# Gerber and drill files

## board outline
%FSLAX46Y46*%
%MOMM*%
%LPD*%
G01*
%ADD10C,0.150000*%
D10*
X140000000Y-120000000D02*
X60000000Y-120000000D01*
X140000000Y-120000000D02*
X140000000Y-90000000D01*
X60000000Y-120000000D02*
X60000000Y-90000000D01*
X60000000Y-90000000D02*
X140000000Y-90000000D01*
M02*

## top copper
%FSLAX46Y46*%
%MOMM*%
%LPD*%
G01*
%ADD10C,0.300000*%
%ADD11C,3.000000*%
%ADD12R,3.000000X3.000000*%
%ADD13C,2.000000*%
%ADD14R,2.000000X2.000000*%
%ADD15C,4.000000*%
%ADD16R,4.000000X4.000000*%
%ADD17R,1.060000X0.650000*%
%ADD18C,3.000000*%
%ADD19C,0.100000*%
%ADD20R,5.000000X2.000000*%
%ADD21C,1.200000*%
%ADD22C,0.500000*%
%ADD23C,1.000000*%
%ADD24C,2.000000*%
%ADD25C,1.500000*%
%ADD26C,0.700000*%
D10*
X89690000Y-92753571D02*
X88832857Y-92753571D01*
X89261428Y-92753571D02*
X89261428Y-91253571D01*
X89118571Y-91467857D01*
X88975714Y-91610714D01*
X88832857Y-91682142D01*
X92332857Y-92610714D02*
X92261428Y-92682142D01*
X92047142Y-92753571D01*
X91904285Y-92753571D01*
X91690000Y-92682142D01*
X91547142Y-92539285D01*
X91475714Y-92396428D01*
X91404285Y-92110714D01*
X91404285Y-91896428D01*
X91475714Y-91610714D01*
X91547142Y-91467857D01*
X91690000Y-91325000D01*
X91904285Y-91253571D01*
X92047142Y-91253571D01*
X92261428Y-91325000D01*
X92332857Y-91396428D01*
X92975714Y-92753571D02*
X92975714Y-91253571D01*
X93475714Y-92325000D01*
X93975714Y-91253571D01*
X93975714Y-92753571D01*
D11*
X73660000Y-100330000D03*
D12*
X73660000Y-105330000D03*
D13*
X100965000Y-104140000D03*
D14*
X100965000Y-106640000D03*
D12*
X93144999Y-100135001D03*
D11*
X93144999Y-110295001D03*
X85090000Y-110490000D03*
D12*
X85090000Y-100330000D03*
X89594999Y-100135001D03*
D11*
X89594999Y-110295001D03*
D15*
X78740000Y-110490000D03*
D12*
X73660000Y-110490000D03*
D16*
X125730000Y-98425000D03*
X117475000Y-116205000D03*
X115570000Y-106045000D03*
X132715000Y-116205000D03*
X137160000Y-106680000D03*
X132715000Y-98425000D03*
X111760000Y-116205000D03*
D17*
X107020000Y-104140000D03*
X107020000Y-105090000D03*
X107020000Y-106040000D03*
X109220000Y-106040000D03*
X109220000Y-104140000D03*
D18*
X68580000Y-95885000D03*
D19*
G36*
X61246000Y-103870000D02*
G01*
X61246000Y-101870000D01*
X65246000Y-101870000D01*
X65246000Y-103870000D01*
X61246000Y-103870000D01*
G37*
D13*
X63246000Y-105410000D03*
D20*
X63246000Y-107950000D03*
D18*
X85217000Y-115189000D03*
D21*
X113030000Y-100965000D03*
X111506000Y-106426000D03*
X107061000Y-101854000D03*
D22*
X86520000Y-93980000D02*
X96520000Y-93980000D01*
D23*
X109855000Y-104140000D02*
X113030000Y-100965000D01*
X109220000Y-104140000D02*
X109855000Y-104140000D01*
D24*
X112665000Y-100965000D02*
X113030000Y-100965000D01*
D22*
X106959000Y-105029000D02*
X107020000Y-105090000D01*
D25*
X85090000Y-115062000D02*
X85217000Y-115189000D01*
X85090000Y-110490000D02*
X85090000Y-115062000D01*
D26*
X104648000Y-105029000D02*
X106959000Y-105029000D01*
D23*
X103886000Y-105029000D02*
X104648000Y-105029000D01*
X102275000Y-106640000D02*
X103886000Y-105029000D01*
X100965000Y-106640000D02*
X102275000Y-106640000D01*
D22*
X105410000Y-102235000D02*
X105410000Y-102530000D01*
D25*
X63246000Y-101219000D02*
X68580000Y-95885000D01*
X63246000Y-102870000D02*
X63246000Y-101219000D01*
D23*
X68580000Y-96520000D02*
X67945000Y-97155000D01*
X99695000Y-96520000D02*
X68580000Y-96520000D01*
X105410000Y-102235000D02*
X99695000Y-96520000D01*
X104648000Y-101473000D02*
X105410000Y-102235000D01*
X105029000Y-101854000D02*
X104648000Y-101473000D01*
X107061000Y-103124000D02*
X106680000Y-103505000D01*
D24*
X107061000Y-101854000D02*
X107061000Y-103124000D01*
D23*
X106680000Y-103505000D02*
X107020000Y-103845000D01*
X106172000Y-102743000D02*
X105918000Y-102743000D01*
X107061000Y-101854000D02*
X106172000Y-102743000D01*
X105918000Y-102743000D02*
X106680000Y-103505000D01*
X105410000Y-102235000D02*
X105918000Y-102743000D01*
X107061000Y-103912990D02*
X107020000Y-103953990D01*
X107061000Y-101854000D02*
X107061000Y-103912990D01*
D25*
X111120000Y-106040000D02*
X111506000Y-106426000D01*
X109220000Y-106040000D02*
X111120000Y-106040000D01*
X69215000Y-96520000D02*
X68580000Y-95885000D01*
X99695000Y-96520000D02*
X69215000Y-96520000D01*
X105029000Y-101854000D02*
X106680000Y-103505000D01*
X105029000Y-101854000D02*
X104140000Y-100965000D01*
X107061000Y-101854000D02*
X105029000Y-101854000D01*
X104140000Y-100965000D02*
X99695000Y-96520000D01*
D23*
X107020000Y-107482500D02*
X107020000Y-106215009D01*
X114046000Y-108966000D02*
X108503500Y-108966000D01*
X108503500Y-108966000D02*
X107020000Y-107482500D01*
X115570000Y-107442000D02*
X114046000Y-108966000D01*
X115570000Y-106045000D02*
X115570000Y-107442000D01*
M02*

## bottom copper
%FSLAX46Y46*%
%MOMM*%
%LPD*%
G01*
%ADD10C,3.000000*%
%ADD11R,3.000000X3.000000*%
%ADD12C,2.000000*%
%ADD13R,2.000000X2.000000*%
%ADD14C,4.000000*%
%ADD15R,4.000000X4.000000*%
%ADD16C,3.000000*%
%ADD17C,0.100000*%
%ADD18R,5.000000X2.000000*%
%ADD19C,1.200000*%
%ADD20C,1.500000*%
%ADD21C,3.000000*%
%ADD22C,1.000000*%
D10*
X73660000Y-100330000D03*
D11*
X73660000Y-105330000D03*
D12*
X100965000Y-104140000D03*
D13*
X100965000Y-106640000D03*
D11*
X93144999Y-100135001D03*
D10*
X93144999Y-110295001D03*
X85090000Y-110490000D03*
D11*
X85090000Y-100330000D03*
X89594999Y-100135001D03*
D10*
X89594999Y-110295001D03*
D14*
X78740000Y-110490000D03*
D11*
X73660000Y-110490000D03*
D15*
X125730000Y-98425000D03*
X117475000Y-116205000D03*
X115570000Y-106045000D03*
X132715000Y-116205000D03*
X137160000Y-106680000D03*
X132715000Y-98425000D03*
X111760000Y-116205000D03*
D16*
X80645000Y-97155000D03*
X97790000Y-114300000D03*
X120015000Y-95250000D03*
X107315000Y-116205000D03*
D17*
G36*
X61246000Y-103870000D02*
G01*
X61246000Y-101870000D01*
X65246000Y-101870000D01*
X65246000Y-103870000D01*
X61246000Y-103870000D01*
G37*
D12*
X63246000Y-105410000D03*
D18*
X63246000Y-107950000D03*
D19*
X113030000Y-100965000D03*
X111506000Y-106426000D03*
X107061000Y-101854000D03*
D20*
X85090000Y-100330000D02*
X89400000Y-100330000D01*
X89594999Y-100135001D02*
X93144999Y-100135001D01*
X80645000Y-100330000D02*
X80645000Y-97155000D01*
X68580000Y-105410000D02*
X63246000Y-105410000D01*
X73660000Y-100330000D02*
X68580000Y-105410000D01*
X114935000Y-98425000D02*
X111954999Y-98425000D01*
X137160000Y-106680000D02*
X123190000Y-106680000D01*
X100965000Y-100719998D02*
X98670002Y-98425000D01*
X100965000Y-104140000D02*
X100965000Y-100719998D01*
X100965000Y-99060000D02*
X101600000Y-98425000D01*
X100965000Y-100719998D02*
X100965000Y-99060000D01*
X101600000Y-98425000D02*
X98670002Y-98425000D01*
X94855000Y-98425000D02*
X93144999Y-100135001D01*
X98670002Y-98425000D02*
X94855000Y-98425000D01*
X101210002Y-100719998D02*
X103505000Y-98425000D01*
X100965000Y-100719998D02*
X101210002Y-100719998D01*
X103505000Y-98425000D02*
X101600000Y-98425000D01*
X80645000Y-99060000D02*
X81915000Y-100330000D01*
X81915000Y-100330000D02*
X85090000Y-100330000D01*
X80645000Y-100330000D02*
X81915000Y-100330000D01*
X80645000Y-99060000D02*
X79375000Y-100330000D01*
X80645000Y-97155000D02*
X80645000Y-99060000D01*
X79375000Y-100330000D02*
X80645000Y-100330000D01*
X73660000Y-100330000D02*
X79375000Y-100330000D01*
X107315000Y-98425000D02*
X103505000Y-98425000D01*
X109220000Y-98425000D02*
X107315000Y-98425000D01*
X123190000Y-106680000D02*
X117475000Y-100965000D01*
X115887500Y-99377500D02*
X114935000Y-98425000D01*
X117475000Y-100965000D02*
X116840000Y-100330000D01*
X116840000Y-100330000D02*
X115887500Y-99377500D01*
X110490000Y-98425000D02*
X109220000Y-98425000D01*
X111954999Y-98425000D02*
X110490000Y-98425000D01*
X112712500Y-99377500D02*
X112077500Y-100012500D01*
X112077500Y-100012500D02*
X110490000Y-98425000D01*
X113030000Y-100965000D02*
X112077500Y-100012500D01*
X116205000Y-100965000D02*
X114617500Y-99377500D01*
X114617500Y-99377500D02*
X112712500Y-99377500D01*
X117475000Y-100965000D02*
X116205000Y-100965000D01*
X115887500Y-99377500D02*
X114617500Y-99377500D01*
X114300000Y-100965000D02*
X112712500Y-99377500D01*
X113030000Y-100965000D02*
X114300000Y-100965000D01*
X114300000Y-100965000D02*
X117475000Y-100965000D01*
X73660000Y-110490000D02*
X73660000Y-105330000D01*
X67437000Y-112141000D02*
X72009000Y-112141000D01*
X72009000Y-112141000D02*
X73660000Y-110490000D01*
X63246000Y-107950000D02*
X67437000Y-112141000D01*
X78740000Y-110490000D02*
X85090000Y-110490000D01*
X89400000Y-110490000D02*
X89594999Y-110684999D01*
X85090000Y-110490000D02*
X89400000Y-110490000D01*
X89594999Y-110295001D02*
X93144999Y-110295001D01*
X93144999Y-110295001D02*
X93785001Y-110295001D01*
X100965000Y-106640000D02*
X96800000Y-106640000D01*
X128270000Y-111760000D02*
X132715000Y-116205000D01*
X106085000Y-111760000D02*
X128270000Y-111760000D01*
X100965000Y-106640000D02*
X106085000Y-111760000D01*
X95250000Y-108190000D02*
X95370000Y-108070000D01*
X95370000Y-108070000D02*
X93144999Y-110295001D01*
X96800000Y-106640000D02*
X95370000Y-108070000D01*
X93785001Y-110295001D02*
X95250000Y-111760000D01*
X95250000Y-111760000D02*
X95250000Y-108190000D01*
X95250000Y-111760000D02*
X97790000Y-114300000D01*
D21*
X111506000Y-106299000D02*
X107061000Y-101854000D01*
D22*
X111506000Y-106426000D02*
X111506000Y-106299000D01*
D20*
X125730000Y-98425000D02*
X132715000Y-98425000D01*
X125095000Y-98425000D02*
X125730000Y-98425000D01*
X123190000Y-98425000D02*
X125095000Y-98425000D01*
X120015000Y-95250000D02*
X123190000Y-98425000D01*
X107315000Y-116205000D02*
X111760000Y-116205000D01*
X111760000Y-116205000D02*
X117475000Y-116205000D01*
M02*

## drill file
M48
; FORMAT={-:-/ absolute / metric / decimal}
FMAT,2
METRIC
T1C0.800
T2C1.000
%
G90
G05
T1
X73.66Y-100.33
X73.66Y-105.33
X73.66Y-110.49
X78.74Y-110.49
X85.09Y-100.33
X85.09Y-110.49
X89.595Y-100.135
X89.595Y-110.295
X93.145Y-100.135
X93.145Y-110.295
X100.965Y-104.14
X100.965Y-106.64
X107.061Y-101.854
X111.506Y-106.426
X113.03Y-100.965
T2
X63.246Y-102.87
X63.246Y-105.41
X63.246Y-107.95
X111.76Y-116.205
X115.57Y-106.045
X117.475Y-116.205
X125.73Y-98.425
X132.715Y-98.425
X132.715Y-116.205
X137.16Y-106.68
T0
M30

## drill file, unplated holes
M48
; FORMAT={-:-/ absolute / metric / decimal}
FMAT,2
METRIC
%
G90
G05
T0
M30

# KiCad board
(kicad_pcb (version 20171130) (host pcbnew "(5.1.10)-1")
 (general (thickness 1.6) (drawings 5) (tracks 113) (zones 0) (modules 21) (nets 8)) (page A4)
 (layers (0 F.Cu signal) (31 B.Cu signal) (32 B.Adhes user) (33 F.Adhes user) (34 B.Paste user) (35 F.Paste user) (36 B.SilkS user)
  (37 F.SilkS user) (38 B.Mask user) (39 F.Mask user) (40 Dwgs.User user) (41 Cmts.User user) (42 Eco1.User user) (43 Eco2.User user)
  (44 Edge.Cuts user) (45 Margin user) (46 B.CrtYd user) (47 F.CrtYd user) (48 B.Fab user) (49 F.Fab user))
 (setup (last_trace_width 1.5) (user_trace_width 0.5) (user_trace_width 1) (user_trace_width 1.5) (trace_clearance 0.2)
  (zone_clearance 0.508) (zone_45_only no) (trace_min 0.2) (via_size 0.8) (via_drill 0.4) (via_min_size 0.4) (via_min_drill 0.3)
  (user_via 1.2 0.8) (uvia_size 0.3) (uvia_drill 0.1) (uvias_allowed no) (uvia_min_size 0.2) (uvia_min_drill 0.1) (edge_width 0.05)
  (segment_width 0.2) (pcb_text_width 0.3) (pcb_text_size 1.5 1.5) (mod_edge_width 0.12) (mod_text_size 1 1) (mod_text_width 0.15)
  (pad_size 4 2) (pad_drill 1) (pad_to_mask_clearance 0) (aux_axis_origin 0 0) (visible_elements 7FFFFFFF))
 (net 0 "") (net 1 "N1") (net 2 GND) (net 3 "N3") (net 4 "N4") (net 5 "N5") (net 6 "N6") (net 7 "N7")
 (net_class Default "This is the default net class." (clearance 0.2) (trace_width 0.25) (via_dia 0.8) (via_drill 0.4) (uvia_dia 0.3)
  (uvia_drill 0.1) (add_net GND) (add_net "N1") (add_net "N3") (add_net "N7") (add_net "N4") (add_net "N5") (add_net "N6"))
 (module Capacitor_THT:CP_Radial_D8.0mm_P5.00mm (layer F.Cu) (at 73.66 100.33 270)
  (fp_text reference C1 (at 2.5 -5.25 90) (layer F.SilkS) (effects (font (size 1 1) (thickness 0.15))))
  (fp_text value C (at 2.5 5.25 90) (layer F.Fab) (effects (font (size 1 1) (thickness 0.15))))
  (pad 1 thru_hole circle (at 0 0 270) (size 3 3) (drill 0.8) (layers *.Cu *.Mask) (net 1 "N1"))
  (pad 2 thru_hole rect (at 5 0 270) (size 3 3) (drill 0.8) (layers *.Cu *.Mask) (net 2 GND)))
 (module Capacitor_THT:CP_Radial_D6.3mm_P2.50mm (layer F.Cu) (at 100.965 104.14 270)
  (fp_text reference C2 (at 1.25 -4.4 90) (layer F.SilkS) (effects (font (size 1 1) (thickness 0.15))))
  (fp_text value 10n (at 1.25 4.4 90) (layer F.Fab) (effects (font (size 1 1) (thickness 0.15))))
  (pad 1 thru_hole circle (at 0 0 270) (size 2 2) (drill 0.8) (layers *.Cu *.Mask) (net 1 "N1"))
  (pad 2 thru_hole rect (at 2.5 0 270) (size 2 2) (drill 0.8) (layers *.Cu *.Mask) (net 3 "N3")))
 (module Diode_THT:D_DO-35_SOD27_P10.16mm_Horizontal (layer F.Cu) (at 93.144999 100.135001 270)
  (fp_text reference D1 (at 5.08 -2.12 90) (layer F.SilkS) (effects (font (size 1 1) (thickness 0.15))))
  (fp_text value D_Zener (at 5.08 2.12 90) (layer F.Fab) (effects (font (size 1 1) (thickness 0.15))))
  (pad 1 thru_hole rect (at 0 0 270) (size 3 3) (drill 0.8) (layers *.Cu *.Mask) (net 1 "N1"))
  (pad 2 thru_hole circle (at 10.16 0 270) (size 3 3) (drill 0.8) (layers *.Cu *.Mask) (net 3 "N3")))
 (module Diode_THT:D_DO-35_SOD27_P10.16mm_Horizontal (layer F.Cu) (at 85.09 100.33 270)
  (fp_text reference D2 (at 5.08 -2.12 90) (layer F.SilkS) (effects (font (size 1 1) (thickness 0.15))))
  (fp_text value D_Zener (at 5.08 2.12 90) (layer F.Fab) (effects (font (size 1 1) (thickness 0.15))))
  (pad 2 thru_hole circle (at 10.16 0 270) (size 3 3) (drill 0.8) (layers *.Cu *.Mask) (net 3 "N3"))
  (pad 1 thru_hole rect (at 0 0 270) (size 3 3) (drill 0.8) (layers *.Cu *.Mask) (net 1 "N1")))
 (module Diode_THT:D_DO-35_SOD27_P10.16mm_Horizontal (layer F.Cu) (at 89.594999 100.135001 270)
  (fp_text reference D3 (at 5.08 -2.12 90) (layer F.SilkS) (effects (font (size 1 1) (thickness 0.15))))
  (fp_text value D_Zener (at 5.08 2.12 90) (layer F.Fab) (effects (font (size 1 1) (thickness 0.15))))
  (pad 1 thru_hole rect (at 0 0 270) (size 3 3) (drill 0.8) (layers *.Cu *.Mask) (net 1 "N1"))
  (pad 2 thru_hole circle (at 10.16 0 270) (size 3 3) (drill 0.8) (layers *.Cu *.Mask) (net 3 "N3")))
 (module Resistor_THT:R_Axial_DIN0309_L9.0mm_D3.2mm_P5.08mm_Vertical (layer F.Cu) (at 78.74 110.49 180)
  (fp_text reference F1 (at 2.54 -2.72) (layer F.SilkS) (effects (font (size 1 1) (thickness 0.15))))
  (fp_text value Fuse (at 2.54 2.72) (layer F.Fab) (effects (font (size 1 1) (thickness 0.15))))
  (pad 1 thru_hole circle (at 0 0 180) (size 4 4) (drill 0.8) (layers *.Cu *.Mask) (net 3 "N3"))
  (pad 2 thru_hole rect (at 5.08 0 180) (size 3 3) (drill 0.8) (layers *.Cu *.Mask) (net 2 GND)))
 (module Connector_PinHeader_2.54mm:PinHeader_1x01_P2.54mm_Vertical (layer F.Cu) (at 125.73 98.425 180)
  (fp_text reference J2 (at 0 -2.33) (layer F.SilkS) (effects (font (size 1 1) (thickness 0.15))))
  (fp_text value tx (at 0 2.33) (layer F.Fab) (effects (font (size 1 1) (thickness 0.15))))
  (pad 1 thru_hole rect (at 0 0 180) (size 4 4) (drill 1) (layers *.Cu *.Mask) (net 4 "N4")))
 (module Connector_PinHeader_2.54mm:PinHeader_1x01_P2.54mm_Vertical (layer F.Cu) (at 117.475 116.205 180)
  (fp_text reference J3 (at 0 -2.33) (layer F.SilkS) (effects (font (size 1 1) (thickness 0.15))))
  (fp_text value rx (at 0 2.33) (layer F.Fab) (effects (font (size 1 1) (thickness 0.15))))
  (pad 1 thru_hole rect (at 0 0 180) (size 4 4) (drill 1) (layers *.Cu *.Mask) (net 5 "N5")))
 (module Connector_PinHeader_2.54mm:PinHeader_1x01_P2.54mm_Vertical (layer F.Cu) (at 115.57 106.045 180)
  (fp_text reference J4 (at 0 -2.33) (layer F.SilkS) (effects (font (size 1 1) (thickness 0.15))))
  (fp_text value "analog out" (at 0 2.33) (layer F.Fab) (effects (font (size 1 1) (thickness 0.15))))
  (pad 1 thru_hole rect (at 0 0 180) (size 4 4) (drill 1) (layers *.Cu *.Mask) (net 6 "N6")))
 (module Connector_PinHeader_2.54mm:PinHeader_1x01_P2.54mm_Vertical (layer F.Cu) (at 132.715 116.205 180)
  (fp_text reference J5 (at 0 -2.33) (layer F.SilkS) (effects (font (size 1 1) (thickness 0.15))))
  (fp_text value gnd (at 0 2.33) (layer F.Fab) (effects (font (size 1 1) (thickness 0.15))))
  (pad 1 thru_hole rect (at 0 0 180) (size 4 4) (drill 1) (layers *.Cu *.Mask) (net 3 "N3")))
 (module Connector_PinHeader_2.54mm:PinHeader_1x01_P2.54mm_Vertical (layer F.Cu) (at 137.16 106.68 180)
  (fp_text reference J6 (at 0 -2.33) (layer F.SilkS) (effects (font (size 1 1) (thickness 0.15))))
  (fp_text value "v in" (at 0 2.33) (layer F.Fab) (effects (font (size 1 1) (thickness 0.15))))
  (pad 1 thru_hole rect (at 0 0 180) (size 4 4) (drill 1) (layers *.Cu *.Mask) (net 1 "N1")))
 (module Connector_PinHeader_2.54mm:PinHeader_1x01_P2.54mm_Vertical (layer F.Cu) (at 132.715 98.425 180)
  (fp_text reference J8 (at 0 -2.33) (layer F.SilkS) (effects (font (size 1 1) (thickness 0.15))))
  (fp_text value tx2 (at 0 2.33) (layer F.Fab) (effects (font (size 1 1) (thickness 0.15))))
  (pad 1 thru_hole rect (at 0 0 180) (size 4 4) (drill 1) (layers *.Cu *.Mask) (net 4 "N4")))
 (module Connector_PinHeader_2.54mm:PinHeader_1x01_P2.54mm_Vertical (layer F.Cu) (at 111.76 116.205 180)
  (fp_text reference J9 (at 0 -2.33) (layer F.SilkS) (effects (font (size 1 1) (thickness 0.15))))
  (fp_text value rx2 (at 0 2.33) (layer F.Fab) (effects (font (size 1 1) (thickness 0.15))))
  (pad 1 thru_hole rect (at 0 0 180) (size 4 4) (drill 1) (layers *.Cu *.Mask) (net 5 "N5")))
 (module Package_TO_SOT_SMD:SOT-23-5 (layer F.Cu) (at 108.12 105.09)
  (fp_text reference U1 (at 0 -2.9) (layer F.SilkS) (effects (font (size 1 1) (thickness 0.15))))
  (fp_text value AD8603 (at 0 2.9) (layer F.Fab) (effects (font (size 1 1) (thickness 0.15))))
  (pad 1 smd rect (at -1.1 -0.95) (size 1.06 0.65) (layers F.Cu F.Paste F.Mask) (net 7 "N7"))
  (pad 2 smd rect (at -1.1 0) (size 1.06 0.65) (layers F.Cu F.Paste F.Mask) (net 3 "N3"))
  (pad 3 smd rect (at -1.1 0.95) (size 1.06 0.65) (layers F.Cu F.Paste F.Mask) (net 6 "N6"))
  (pad 4 smd rect (at 1.1 0.95) (size 1.06 0.65) (layers F.Cu F.Paste F.Mask) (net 7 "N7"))
  (pad 5 smd rect (at 1.1 -0.95) (size 1.06 0.65) (layers F.Cu F.Paste F.Mask) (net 1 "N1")))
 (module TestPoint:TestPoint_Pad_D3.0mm (layer B.Cu) (at 80.645 97.155 180)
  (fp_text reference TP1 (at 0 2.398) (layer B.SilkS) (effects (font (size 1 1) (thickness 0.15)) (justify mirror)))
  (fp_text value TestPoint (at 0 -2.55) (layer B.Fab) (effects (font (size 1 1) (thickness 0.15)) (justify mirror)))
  (pad 1 smd circle (at 0 0 180) (size 3 3) (layers B.Cu B.Mask) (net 1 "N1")))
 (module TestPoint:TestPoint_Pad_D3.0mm (layer F.Cu) (at 68.58 95.885 180)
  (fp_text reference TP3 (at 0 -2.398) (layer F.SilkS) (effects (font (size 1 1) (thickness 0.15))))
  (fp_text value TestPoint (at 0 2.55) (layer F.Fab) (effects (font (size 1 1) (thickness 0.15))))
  (pad 1 smd circle (at 0 0 180) (size 3 3) (layers F.Cu F.Mask) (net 7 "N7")))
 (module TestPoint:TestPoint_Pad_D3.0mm (layer B.Cu) (at 97.79 114.3 180)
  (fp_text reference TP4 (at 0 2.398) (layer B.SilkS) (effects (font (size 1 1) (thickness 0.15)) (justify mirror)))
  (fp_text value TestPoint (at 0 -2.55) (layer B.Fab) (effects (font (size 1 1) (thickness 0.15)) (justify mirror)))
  (pad 1 smd circle (at 0 0 180) (size 3 3) (layers B.Cu B.Mask) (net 3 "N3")))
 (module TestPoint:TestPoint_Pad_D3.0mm (layer B.Cu) (at 120.015 95.25 180)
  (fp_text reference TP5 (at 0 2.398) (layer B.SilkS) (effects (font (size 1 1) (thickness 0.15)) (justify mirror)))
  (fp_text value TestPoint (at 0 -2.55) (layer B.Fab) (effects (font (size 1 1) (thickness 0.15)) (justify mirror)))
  (pad 1 smd circle (at 0 0 180) (size 3 3) (layers B.Cu B.Mask) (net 4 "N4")))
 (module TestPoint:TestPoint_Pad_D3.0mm (layer B.Cu) (at 107.315 116.205 180)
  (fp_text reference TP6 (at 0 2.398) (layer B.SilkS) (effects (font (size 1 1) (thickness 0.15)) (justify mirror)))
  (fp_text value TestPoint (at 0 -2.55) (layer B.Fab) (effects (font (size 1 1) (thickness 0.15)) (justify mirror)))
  (pad 1 smd circle (at 0 0 180) (size 3 3) (layers B.Cu B.Mask) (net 5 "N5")))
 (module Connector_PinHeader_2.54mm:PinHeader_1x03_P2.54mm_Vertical (layer F.Cu) (at 63.246 102.87)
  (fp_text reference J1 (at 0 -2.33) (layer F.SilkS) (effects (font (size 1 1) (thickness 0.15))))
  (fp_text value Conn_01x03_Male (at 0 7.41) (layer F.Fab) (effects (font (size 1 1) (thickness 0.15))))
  (pad 1 thru_hole trapezoid (at 0 0) (size 4 2) (drill 1) (layers *.Cu *.Mask) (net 7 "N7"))
  (pad 2 thru_hole circle (at 0 2.54) (size 2 2) (drill 1) (layers *.Cu *.Mask) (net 1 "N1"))
  (pad 3 thru_hole rect (at 0 5.08) (size 5 2) (drill 1) (layers *.Cu *.Mask) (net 2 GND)))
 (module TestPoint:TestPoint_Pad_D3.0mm (layer F.Cu) (at 85.217 115.189)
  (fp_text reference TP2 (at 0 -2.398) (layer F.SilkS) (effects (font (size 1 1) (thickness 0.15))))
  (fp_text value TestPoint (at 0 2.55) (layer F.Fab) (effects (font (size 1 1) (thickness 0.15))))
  (pad 1 smd circle (at 0 0) (size 3 3) (layers F.Cu F.Mask) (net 3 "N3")))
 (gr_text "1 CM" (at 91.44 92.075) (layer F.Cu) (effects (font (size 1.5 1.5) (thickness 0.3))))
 (gr_line (start 140 120) (end 60 120) (layer Edge.Cuts) (width 0.15))
 (gr_line (start 140 120) (end 140 90) (layer Edge.Cuts) (width 0.15))
 (gr_line (start 60 120) (end 60 90) (layer Edge.Cuts) (width 0.15))
 (gr_line (start 60 90) (end 140 90) (layer Edge.Cuts) (width 0.15))
 (segment (start 86.52 93.98) (end 96.52 93.98) (width 0.5) (layer F.Cu) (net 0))
 (segment (start 85.09 100.33) (end 89.4 100.33) (width 1.5) (layer B.Cu) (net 1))
 (segment (start 89.594999 100.135001) (end 93.144999 100.135001) (width 1.5) (layer B.Cu) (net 1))
 (segment (start 80.645 100.33) (end 80.645 97.155) (width 1.5) (layer B.Cu) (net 1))
 (via (at 113.03 100.965) (size 1.2) (drill 0.8) (layers F.Cu B.Cu) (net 1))
 (segment (start 68.58 105.41) (end 63.246 105.41) (width 1.5) (layer B.Cu) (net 1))
 (segment (start 73.66 100.33) (end 68.58 105.41) (width 1.5) (layer B.Cu) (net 1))
 (segment (start 114.935 98.425) (end 111.954999 98.425) (width 1.5) (layer B.Cu) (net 1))
 (segment (start 137.16 106.68) (end 123.19 106.68) (width 1.5) (layer B.Cu) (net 1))
 (segment (start 100.965 100.719998) (end 98.670002 98.425) (width 1.5) (layer B.Cu) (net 1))
 (segment (start 100.965 104.14) (end 100.965 100.719998) (width 1.5) (layer B.Cu) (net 1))
 (segment (start 100.965 99.06) (end 101.6 98.425) (width 1.5) (layer B.Cu) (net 1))
 (segment (start 100.965 100.719998) (end 100.965 99.06) (width 1.5) (layer B.Cu) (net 1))
 (segment (start 101.6 98.425) (end 98.670002 98.425) (width 1.5) (layer B.Cu) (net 1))
 (segment (start 94.855 98.425) (end 93.144999 100.135001) (width 1.5) (layer B.Cu) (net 1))
 (segment (start 98.670002 98.425) (end 94.855 98.425) (width 1.5) (layer B.Cu) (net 1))
 (segment (start 101.210002 100.719998) (end 103.505 98.425) (width 1.5) (layer B.Cu) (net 1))
 (segment (start 100.965 100.719998) (end 101.210002 100.719998) (width 1.5) (layer B.Cu) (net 1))
 (segment (start 103.505 98.425) (end 101.6 98.425) (width 1.5) (layer B.Cu) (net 1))
 (segment (start 80.645 99.06) (end 81.915 100.33) (width 1.5) (layer B.Cu) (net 1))
 (segment (start 81.915 100.33) (end 85.09 100.33) (width 1.5) (layer B.Cu) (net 1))
 (segment (start 80.645 100.33) (end 81.915 100.33) (width 1.5) (layer B.Cu) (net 1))
 (segment (start 80.645 99.06) (end 79.375 100.33) (width 1.5) (layer B.Cu) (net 1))
 (segment (start 80.645 97.155) (end 80.645 99.06) (width 1.5) (layer B.Cu) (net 1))
 (segment (start 79.375 100.33) (end 80.645 100.33) (width 1.5) (layer B.Cu) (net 1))
 (segment (start 73.66 100.33) (end 79.375 100.33) (width 1.5) (layer B.Cu) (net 1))
 (segment (start 107.315 98.425) (end 103.505 98.425) (width 1.5) (layer B.Cu) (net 1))
 (segment (start 109.22 98.425) (end 107.315 98.425) (width 1.5) (layer B.Cu) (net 1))
 (segment (start 123.19 106.68) (end 117.475 100.965) (width 1.5) (layer B.Cu) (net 1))
 (segment (start 115.8875 99.3775) (end 114.935 98.425) (width 1.5) (layer B.Cu) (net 1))
 (segment (start 117.475 100.965) (end 116.84 100.33) (width 1.5) (layer B.Cu) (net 1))
 (segment (start 116.84 100.33) (end 115.8875 99.3775) (width 1.5) (layer B.Cu) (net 1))
 (segment (start 110.49 98.425) (end 109.22 98.425) (width 1.5) (layer B.Cu) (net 1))
 (segment (start 111.954999 98.425) (end 110.49 98.425) (width 1.5) (layer B.Cu) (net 1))
 (segment (start 112.7125 99.3775) (end 112.0775 100.0125) (width 1.5) (layer B.Cu) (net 1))
 (segment (start 112.0775 100.0125) (end 110.49 98.425) (width 1.5) (layer B.Cu) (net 1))
 (segment (start 113.03 100.965) (end 112.0775 100.0125) (width 1.5) (layer B.Cu) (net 1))
 (segment (start 116.205 100.965) (end 114.6175 99.3775) (width 1.5) (layer B.Cu) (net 1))
 (segment (start 114.6175 99.3775) (end 112.7125 99.3775) (width 1.5) (layer B.Cu) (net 1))
 (segment (start 117.475 100.965) (end 116.205 100.965) (width 1.5) (layer B.Cu) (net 1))
 (segment (start 115.8875 99.3775) (end 114.6175 99.3775) (width 1.5) (layer B.Cu) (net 1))
 (segment (start 114.3 100.965) (end 112.7125 99.3775) (width 1.5) (layer B.Cu) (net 1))
 (segment (start 113.03 100.965) (end 114.3 100.965) (width 1.5) (layer B.Cu) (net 1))
 (segment (start 114.3 100.965) (end 117.475 100.965) (width 1.5) (layer B.Cu) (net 1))
 (segment (start 109.855 104.14) (end 113.03 100.965) (width 1) (layer F.Cu) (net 1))
 (segment (start 109.22 104.14) (end 109.855 104.14) (width 1) (layer F.Cu) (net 1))
 (segment (start 112.665 100.965) (end 113.03 100.965) (width 2) (layer F.Cu) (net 1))
 (segment (start 73.66 110.49) (end 73.66 105.33) (width 1.5) (layer B.Cu) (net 2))
 (segment (start 67.437 112.141) (end 72.009 112.141) (width 1.5) (layer B.Cu) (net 2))
 (segment (start 72.009 112.141) (end 73.66 110.49) (width 1.5) (layer B.Cu) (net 2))
 (segment (start 63.246 107.95) (end 67.437 112.141) (width 1.5) (layer B.Cu) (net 2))
 (segment (start 78.74 110.49) (end 85.09 110.49) (width 1.5) (layer B.Cu) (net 3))
 (segment (start 89.4 110.49) (end 89.594999 110.684999) (width 1.5) (layer B.Cu) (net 3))
 (segment (start 85.09 110.49) (end 89.4 110.49) (width 1.5) (layer B.Cu) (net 3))
 (segment (start 89.594999 110.295001) (end 93.144999 110.295001) (width 1.5) (layer B.Cu) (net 3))
 (segment (start 93.144999 110.295001) (end 93.785001 110.295001) (width 1.5) (layer B.Cu) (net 3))
 (segment (start 100.965 106.64) (end 96.8 106.64) (width 1.5) (layer B.Cu) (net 3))
 (segment (start 128.27 111.76) (end 132.715 116.205) (width 1.5) (layer B.Cu) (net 3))
 (segment (start 106.085 111.76) (end 128.27 111.76) (width 1.5) (layer B.Cu) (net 3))
 (segment (start 100.965 106.64) (end 106.085 111.76) (width 1.5) (layer B.Cu) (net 3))
 (segment (start 106.959 105.029) (end 107.02 105.09) (width 0.5) (layer F.Cu) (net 3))
 (segment (start 85.09 115.062) (end 85.217 115.189) (width 1.5) (layer F.Cu) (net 3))
 (segment (start 85.09 110.49) (end 85.09 115.062) (width 1.5) (layer F.Cu) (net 3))
 (segment (start 104.648 105.029) (end 106.959 105.029) (width 0.7) (layer F.Cu) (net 3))
 (segment (start 103.886 105.029) (end 104.648 105.029) (width 1) (layer F.Cu) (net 3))
 (segment (start 102.275 106.64) (end 103.886 105.029) (width 1) (layer F.Cu) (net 3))
 (segment (start 100.965 106.64) (end 102.275 106.64) (width 1) (layer F.Cu) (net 3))
 (segment (start 95.25 108.19) (end 95.37 108.07) (width 1.5) (layer B.Cu) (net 3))
 (segment (start 95.37 108.07) (end 93.144999 110.295001) (width 1.5) (layer B.Cu) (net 3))
 (segment (start 96.8 106.64) (end 95.37 108.07) (width 1.5) (layer B.Cu) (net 3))
 (segment (start 93.785001 110.295001) (end 95.25 111.76) (width 1.5) (layer B.Cu) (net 3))
 (segment (start 95.25 111.76) (end 95.25 108.19) (width 1.5) (layer B.Cu) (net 3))
 (segment (start 95.25 111.76) (end 97.79 114.3) (width 1.5) (layer B.Cu) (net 3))
 (segment (start 105.41 102.235) (end 105.41 102.53) (width 0.5) (layer F.Cu) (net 7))
 (segment (start 63.246 101.219) (end 68.58 95.885) (width 1.5) (layer F.Cu) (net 7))
 (segment (start 63.246 102.87) (end 63.246 101.219) (width 1.5) (layer F.Cu) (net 7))
 (segment (start 68.58 96.52) (end 67.945 97.155) (width 1) (layer F.Cu) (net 7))
 (segment (start 99.695 96.52) (end 68.58 96.52) (width 1) (layer F.Cu) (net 7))
 (segment (start 105.41 102.235) (end 99.695 96.52) (width 1) (layer F.Cu) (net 7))
 (via (at 111.506 106.426) (size 1.2) (drill 0.8) (layers F.Cu B.Cu) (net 7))
 (via (at 107.061 101.854) (size 1.2) (drill 0.8) (layers F.Cu B.Cu) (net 7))
 (segment (start 111.506 106.299) (end 107.061 101.854) (width 3) (layer B.Cu) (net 7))
 (segment (start 111.506 106.426) (end 111.506 106.299) (width 1) (layer B.Cu) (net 7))
 (segment (start 104.648 101.473) (end 105.41 102.235) (width 1) (layer F.Cu) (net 7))
 (segment (start 105.029 101.854) (end 104.648 101.473) (width 1) (layer F.Cu) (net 7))
 (segment (start 107.061 103.124) (end 106.68 103.505) (width 1) (layer F.Cu) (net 7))
 (segment (start 107.061 101.854) (end 107.061 103.124) (width 2) (layer F.Cu) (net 7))
 (segment (start 106.68 103.505) (end 107.02 103.845) (width 1) (layer F.Cu) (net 7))
 (segment (start 106.172 102.743) (end 105.918 102.743) (width 1) (layer F.Cu) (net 7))
 (segment (start 107.061 101.854) (end 106.172 102.743) (width 1) (layer F.Cu) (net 7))
 (segment (start 105.918 102.743) (end 106.68 103.505) (width 1) (layer F.Cu) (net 7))
 (segment (start 105.41 102.235) (end 105.918 102.743) (width 1) (layer F.Cu) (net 7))
 (segment (start 107.061 103.91299) (end 107.02 103.95399) (width 1) (layer F.Cu) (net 7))
 (segment (start 107.061 101.854) (end 107.061 103.91299) (width 1) (layer F.Cu) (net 7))
 (segment (start 111.12 106.04) (end 111.506 106.426) (width 1.5) (layer F.Cu) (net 7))
 (segment (start 109.22 106.04) (end 111.12 106.04) (width 1.5) (layer F.Cu) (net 7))
 (segment (start 69.215 96.52) (end 68.58 95.885) (width 1.5) (layer F.Cu) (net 7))
 (segment (start 99.695 96.52) (end 69.215 96.52) (width 1.5) (layer F.Cu) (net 7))
 (segment (start 105.029 101.854) (end 106.68 103.505) (width 1.5) (layer F.Cu) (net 7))
 (segment (start 105.029 101.854) (end 104.14 100.965) (width 1.5) (layer F.Cu) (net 7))
 (segment (start 107.061 101.854) (end 105.029 101.854) (width 1.5) (layer F.Cu) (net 7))
 (segment (start 104.14 100.965) (end 99.695 96.52) (width 1.5) (layer F.Cu) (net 7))
 (segment (start 125.73 98.425) (end 132.715 98.425) (width 1.5) (layer B.Cu) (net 4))
 (segment (start 125.095 98.425) (end 125.73 98.425) (width 1.5) (layer B.Cu) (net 4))
 (segment (start 123.19 98.425) (end 125.095 98.425) (width 1.5) (layer B.Cu) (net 4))
 (segment (start 120.015 95.25) (end 123.19 98.425) (width 1.5) (layer B.Cu) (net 4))
 (segment (start 107.315 116.205) (end 111.76 116.205) (width 1.5) (layer B.Cu) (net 5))
 (segment (start 111.76 116.205) (end 117.475 116.205) (width 1.5) (layer B.Cu) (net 5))
 (segment (start 107.02 107.4825) (end 107.02 106.215009) (width 1) (layer F.Cu) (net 6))
 (segment (start 114.046 108.966) (end 108.5035 108.966) (width 1) (layer F.Cu) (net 6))
 (segment (start 108.5035 108.966) (end 107.02 107.4825) (width 1) (layer F.Cu) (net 6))
 (segment (start 115.57 107.442) (end 114.046 108.966) (width 1) (layer F.Cu) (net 6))
 (segment (start 115.57 106.045) (end 115.57 107.442) (width 1) (layer F.Cu) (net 6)))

